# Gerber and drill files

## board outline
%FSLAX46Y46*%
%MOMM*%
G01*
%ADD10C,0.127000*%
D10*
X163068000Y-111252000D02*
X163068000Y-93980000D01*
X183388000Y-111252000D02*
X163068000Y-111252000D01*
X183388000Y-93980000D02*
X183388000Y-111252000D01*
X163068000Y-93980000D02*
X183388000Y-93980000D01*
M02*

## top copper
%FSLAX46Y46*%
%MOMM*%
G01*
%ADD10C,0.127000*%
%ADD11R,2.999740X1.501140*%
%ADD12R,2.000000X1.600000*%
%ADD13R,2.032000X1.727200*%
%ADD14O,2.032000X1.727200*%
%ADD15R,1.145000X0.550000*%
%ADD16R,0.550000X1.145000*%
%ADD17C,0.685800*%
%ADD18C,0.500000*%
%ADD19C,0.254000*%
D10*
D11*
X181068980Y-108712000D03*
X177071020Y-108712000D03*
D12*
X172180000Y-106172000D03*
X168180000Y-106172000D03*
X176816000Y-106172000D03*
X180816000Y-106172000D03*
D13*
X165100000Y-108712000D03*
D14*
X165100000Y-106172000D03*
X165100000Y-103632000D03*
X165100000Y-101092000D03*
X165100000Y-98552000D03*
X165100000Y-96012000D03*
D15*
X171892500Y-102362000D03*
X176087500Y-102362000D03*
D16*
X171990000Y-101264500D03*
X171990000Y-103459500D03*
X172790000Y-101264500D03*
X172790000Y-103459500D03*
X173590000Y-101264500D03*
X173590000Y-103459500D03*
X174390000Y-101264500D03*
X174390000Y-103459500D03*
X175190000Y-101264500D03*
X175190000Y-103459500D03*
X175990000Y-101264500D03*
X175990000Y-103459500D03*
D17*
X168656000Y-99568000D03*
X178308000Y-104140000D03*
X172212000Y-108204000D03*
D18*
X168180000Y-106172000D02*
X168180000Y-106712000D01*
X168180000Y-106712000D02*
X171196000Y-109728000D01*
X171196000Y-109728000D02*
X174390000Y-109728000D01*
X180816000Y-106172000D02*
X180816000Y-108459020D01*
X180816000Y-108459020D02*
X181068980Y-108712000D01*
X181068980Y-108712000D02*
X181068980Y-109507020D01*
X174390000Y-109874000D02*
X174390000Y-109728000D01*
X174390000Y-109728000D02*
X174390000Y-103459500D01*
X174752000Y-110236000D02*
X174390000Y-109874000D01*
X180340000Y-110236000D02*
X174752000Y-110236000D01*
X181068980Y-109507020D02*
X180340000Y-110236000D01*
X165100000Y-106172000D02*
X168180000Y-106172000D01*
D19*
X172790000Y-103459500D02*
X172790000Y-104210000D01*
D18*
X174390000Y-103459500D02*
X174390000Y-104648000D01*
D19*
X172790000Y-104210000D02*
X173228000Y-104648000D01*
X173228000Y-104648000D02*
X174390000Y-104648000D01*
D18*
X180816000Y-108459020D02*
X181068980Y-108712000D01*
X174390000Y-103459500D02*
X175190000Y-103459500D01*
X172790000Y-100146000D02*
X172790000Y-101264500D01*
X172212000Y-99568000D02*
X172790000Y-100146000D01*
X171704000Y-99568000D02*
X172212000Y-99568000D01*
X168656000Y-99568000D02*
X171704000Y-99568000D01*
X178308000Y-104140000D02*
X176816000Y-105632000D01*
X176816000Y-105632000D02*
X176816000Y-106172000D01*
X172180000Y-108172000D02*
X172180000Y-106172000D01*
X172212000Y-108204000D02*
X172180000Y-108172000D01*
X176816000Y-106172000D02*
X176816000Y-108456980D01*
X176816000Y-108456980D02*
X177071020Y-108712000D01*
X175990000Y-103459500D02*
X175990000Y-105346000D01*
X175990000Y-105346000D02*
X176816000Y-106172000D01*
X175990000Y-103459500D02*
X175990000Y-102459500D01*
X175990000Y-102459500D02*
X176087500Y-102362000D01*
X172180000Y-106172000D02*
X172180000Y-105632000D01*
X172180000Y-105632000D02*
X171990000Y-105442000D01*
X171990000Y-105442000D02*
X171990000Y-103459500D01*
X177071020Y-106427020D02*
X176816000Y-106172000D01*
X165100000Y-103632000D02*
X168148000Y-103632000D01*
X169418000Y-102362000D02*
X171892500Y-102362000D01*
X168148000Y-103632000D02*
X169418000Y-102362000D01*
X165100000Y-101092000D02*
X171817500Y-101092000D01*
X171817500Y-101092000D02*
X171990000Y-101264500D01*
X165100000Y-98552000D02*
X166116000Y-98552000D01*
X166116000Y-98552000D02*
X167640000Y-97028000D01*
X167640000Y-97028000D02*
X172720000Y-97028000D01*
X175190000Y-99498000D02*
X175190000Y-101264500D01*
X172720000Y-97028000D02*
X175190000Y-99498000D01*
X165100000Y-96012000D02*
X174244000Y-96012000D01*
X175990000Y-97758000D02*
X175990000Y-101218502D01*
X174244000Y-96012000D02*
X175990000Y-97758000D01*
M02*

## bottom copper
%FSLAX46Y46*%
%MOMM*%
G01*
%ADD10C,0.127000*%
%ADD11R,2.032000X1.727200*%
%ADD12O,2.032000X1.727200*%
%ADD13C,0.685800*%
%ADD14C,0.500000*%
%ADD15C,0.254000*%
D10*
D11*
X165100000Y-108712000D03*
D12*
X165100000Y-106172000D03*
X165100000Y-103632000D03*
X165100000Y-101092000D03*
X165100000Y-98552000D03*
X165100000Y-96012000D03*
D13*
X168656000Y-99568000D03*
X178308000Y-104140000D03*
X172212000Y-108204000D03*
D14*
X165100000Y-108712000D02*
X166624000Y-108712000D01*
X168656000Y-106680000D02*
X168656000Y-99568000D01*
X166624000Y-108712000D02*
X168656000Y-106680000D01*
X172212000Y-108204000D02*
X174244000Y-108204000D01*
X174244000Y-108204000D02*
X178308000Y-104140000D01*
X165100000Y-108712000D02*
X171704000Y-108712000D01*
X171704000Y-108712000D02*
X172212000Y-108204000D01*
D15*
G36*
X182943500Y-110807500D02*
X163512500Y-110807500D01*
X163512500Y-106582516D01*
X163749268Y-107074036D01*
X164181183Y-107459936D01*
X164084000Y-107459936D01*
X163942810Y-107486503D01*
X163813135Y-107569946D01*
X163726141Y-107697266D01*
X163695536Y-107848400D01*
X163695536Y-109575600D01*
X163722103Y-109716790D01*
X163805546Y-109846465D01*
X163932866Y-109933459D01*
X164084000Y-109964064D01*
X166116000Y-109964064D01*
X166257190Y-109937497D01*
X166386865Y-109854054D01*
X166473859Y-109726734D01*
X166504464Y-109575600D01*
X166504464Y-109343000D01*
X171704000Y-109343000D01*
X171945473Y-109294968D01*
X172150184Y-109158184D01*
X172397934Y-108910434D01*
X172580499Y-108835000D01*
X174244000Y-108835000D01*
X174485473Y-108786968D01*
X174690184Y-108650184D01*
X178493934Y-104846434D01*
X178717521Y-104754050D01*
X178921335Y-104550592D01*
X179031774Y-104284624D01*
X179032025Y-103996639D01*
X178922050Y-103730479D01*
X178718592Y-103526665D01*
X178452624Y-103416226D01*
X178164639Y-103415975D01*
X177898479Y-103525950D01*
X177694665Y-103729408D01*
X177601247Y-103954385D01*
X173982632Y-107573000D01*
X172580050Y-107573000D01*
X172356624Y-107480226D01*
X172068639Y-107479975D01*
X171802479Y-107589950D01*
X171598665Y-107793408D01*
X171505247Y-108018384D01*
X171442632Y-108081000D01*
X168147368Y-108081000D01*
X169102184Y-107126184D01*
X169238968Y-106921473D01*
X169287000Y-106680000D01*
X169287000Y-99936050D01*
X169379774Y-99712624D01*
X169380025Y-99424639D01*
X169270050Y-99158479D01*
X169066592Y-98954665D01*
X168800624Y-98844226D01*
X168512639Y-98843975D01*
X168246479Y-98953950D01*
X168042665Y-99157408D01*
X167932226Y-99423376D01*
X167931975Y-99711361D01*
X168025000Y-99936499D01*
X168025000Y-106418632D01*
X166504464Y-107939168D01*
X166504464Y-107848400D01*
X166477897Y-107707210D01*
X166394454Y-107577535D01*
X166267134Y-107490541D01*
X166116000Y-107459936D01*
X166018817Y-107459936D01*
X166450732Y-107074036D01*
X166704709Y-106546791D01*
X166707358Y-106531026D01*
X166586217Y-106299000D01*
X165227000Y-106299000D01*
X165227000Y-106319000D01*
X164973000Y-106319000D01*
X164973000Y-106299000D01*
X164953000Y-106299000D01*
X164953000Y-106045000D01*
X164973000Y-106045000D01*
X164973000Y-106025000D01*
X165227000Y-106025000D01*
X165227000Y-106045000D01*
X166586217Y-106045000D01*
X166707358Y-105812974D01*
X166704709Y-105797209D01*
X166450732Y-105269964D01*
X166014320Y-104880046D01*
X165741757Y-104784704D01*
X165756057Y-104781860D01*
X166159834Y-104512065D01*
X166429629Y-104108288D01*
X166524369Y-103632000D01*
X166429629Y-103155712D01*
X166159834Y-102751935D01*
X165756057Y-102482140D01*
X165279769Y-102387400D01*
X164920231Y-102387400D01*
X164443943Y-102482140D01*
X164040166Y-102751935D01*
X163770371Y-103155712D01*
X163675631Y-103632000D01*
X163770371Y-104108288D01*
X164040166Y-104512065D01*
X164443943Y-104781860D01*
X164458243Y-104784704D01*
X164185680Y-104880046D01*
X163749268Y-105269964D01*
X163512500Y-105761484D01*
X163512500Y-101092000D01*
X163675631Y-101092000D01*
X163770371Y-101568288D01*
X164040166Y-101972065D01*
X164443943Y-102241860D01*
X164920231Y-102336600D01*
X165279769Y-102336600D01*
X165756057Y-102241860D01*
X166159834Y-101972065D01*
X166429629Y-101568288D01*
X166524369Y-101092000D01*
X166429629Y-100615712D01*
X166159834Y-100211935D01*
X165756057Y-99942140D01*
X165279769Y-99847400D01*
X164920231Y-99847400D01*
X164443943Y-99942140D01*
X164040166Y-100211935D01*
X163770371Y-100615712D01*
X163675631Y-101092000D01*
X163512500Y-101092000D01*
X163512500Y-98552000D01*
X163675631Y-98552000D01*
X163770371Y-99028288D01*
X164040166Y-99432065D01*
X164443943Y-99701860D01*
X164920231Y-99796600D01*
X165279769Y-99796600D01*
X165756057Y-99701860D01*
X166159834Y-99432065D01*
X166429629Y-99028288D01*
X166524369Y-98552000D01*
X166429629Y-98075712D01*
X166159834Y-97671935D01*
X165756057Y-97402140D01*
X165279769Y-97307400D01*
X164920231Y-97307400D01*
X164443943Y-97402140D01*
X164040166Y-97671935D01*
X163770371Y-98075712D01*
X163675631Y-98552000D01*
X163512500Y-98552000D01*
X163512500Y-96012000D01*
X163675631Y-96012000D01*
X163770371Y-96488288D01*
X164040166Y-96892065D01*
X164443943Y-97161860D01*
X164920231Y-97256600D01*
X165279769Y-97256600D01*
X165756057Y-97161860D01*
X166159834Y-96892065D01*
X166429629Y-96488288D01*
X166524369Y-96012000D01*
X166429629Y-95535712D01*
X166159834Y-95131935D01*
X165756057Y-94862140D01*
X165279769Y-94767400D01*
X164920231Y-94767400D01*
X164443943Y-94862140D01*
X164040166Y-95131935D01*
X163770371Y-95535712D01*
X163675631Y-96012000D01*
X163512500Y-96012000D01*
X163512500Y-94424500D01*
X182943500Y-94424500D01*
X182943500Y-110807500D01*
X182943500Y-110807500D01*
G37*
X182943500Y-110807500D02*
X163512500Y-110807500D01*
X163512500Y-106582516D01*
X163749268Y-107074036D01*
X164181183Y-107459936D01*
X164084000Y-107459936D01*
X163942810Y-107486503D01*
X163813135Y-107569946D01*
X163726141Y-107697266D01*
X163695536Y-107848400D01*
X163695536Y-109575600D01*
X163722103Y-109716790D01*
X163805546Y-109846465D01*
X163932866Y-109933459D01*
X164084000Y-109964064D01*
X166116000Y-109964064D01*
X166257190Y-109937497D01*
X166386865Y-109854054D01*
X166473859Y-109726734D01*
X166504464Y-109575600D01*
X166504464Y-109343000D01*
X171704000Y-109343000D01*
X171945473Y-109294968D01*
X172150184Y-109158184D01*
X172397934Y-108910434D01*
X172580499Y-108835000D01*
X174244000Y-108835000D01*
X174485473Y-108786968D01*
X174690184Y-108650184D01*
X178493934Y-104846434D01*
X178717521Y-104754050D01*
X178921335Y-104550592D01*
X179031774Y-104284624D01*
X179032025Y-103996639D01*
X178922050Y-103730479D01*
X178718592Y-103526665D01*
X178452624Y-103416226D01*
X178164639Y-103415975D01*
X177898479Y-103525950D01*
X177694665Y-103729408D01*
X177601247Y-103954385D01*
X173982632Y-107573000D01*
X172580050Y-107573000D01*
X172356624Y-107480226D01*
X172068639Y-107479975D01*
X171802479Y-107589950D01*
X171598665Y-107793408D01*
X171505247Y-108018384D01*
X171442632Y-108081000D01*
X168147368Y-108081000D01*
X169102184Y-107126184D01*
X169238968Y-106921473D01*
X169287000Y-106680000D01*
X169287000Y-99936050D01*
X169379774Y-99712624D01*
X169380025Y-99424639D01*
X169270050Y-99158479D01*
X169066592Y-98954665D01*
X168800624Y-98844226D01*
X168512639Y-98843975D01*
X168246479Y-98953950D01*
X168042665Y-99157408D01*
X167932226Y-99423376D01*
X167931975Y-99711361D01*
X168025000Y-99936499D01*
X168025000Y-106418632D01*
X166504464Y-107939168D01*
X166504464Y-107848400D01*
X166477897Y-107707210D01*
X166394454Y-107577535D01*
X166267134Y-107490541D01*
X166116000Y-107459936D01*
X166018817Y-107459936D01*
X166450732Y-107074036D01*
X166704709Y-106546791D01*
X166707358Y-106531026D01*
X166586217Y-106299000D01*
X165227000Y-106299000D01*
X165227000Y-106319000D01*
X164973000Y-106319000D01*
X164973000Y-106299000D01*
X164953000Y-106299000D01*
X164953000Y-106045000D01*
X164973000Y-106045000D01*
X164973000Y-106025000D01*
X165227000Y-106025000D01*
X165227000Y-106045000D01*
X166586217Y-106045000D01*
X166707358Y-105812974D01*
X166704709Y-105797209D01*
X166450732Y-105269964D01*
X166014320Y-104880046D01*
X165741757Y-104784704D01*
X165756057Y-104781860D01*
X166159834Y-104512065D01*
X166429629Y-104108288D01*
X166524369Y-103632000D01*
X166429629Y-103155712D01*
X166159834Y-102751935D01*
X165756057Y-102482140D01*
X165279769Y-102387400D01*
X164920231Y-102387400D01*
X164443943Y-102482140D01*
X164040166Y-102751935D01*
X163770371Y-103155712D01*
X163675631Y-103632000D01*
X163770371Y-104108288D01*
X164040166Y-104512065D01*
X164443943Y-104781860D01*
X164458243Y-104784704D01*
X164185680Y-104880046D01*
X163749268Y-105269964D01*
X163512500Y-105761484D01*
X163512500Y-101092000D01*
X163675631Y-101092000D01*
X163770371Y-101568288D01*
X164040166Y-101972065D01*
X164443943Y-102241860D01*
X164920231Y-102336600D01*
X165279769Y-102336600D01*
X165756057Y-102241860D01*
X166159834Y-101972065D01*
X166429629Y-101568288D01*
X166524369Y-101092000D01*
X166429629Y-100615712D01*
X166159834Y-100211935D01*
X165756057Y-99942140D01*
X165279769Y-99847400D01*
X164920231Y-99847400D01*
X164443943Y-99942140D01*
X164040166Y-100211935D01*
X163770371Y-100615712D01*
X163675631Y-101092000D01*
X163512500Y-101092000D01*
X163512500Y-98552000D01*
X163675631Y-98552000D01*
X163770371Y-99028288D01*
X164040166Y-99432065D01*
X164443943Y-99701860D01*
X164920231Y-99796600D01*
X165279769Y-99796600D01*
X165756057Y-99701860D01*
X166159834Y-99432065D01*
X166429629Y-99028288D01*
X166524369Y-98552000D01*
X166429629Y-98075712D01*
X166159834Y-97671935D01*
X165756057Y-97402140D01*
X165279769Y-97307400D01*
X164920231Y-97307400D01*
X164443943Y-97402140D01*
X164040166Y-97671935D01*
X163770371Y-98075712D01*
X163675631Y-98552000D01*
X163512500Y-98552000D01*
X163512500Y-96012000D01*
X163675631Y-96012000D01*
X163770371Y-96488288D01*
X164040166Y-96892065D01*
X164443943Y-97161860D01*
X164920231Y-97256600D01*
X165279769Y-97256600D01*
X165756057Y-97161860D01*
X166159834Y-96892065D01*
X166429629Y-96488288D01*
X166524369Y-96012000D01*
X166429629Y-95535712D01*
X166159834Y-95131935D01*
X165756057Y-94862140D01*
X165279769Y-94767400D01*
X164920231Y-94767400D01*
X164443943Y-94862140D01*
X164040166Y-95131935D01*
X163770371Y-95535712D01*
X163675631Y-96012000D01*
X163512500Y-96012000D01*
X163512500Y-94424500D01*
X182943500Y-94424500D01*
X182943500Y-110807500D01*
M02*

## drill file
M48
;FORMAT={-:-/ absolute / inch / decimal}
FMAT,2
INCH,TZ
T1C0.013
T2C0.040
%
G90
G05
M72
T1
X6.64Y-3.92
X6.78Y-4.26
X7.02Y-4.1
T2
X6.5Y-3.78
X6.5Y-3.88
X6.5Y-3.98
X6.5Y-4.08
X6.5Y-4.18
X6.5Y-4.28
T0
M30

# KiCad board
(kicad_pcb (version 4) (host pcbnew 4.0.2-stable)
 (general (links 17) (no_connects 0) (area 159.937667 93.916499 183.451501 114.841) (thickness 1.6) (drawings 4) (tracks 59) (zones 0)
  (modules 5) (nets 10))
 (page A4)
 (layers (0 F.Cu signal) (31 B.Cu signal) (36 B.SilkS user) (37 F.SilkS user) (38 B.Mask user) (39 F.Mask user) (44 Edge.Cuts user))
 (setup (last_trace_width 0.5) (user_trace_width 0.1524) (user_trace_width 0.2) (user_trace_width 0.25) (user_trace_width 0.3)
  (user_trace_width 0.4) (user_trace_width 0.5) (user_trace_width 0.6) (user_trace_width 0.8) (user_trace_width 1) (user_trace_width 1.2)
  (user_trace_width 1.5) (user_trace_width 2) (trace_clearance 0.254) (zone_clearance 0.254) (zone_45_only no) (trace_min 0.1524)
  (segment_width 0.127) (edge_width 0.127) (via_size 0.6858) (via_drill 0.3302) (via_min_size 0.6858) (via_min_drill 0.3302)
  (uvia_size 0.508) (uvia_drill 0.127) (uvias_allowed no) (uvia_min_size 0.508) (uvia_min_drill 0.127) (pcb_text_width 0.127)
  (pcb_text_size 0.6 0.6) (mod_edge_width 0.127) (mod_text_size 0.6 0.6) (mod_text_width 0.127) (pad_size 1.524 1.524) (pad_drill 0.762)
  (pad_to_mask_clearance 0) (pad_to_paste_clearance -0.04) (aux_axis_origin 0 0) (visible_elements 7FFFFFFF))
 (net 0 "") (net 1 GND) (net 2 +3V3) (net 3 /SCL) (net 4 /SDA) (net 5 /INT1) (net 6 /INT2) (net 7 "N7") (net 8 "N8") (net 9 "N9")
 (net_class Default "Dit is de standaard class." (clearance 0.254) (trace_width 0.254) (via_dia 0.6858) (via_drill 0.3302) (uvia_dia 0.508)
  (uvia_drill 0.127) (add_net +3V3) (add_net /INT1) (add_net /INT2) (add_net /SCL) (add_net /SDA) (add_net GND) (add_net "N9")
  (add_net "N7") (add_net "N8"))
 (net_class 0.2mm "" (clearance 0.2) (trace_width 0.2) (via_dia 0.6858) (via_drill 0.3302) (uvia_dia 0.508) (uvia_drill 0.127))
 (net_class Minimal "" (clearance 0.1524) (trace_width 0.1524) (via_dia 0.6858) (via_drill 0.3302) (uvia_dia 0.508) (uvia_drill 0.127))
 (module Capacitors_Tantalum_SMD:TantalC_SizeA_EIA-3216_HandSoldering (layer F.Cu) (at 179.07 108.712)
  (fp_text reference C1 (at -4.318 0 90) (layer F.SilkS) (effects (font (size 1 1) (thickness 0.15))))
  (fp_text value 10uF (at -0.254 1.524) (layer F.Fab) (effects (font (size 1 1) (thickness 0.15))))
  (pad 2 smd rect (at 1.99898 0) (size 2.99974 1.50114) (layers F.Cu F.Mask) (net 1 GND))
  (pad 1 smd rect (at -1.99898 0) (size 2.99974 1.50114) (layers F.Cu F.Mask) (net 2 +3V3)))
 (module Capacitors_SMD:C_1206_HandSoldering (layer F.Cu) (at 170.18 106.172 180)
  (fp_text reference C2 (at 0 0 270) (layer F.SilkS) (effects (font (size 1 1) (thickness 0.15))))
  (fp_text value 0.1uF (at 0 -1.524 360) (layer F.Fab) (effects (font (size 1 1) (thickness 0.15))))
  (pad 1 smd rect (at -2 0 180) (size 2 1.6) (layers F.Cu F.Mask) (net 2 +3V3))
  (pad 2 smd rect (at 2 0 180) (size 2 1.6) (layers F.Cu F.Mask) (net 1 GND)))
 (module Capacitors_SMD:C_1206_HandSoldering (layer F.Cu) (at 178.816 106.172)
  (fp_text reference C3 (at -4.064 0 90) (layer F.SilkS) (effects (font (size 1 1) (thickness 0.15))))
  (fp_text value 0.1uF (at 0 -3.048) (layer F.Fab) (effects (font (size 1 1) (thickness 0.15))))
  (pad 1 smd rect (at -2 0) (size 2 1.6) (layers F.Cu F.Mask) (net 2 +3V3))
  (pad 2 smd rect (at 2 0) (size 2 1.6) (layers F.Cu F.Mask) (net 1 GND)))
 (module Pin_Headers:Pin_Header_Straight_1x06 (layer F.Cu) (at 165.1 108.712 180)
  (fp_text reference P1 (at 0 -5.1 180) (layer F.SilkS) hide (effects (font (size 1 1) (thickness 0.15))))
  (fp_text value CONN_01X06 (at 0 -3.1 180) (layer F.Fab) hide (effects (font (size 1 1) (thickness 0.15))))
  (pad 1 thru_hole rect (at 0 0 180) (size 2.032 1.7272) (drill 1.016) (layers *.Cu *.Mask F.SilkS) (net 2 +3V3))
  (pad 2 thru_hole oval (at 0 2.54 180) (size 2.032 1.7272) (drill 1.016) (layers *.Cu *.Mask F.SilkS) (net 1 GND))
  (pad 3 thru_hole oval (at 0 5.08 180) (size 2.032 1.7272) (drill 1.016) (layers *.Cu *.Mask F.SilkS) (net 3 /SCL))
  (pad 4 thru_hole oval (at 0 7.62 180) (size 2.032 1.7272) (drill 1.016) (layers *.Cu *.Mask F.SilkS) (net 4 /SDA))
  (pad 5 thru_hole oval (at 0 10.16 180) (size 2.032 1.7272) (drill 1.016) (layers *.Cu *.Mask F.SilkS) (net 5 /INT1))
  (pad 6 thru_hole oval (at 0 12.7 180) (size 2.032 1.7272) (drill 1.016) (layers *.Cu *.Mask F.SilkS) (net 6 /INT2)))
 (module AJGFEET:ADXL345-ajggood (layer F.Cu) (at 173.99 102.362)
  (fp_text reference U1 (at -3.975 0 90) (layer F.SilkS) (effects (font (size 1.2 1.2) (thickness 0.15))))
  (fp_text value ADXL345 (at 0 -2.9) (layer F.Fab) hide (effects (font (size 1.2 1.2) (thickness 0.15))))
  (pad 14 smd rect (at -2.0975 0) (size 1.145 0.55) (layers F.Cu F.Mask) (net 3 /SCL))
  (pad 7 smd rect (at 2.0975 0) (size 1.145 0.55) (layers F.Cu F.Mask) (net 2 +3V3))
  (pad 13 smd rect (at -2 -1.0975) (size 0.55 1.145) (layers F.Cu F.Mask) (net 4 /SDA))
  (pad 1 smd rect (at -2 1.0975) (size 0.55 1.145) (layers F.Cu F.Mask) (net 2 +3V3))
  (pad 12 smd rect (at -1.2 -1.0975) (size 0.55 1.145) (layers F.Cu F.Mask) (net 2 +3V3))
  (pad 2 smd rect (at -1.2 1.0975) (size 0.55 1.145) (layers F.Cu F.Mask) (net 1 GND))
  (pad 11 smd rect (at -0.4 -1.0975) (size 0.55 1.145) (layers F.Cu F.Mask) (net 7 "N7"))
  (pad 3 smd rect (at -0.4 1.0975) (size 0.55 1.145) (layers F.Cu F.Mask) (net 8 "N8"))
  (pad 10 smd rect (at 0.4 -1.0975) (size 0.55 1.145) (layers F.Cu F.Mask) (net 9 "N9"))
  (pad 4 smd rect (at 0.4 1.0975) (size 0.55 1.145) (layers F.Cu F.Mask) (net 1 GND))
  (pad 9 smd rect (at 1.2 -1.0975) (size 0.55 1.145) (layers F.Cu F.Mask) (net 5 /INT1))
  (pad 5 smd rect (at 1.2 1.0975) (size 0.55 1.145) (layers F.Cu F.Mask) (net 1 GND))
  (pad 8 smd rect (at 2 -1.0975) (size 0.55 1.145) (layers F.Cu F.Mask) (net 6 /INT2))
  (pad 6 smd rect (at 2 1.0975) (size 0.55 1.145) (layers F.Cu F.Mask) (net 2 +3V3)))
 (gr_line (start 163.068 111.252) (end 163.068 93.98) (angle 90) (layer Edge.Cuts) (width 0.127))
 (gr_line (start 183.388 111.252) (end 163.068 111.252) (angle 90) (layer Edge.Cuts) (width 0.127))
 (gr_line (start 183.388 93.98) (end 183.388 111.252) (angle 90) (layer Edge.Cuts) (width 0.127))
 (gr_line (start 163.068 93.98) (end 183.388 93.98) (angle 90) (layer Edge.Cuts) (width 0.127))
 (segment (start 168.18 106.172) (end 168.18 106.712) (width 0.5) (layer F.Cu) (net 1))
 (segment (start 168.18 106.712) (end 171.196 109.728) (width 0.5) (layer F.Cu) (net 1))
 (segment (start 171.196 109.728) (end 174.39 109.728) (width 0.5) (layer F.Cu) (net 1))
 (segment (start 180.816 106.172) (end 180.816 108.45902) (width 0.5) (layer F.Cu) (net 1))
 (segment (start 180.816 108.45902) (end 181.06898 108.712) (width 0.5) (layer F.Cu) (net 1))
 (segment (start 181.06898 108.712) (end 181.06898 109.50702) (width 0.5) (layer F.Cu) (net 1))
 (segment (start 174.39 109.874) (end 174.39 109.728) (width 0.5) (layer F.Cu) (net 1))
 (segment (start 174.39 109.728) (end 174.39 103.4595) (width 0.5) (layer F.Cu) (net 1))
 (segment (start 174.752 110.236) (end 174.39 109.874) (width 0.5) (layer F.Cu) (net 1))
 (segment (start 180.34 110.236) (end 174.752 110.236) (width 0.5) (layer F.Cu) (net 1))
 (segment (start 181.06898 109.50702) (end 180.34 110.236) (width 0.5) (layer F.Cu) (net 1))
 (segment (start 165.1 106.172) (end 168.18 106.172) (width 0.5) (layer F.Cu) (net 1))
 (segment (start 172.79 103.4595) (end 172.79 104.21) (width 0.254) (layer F.Cu) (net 1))
 (segment (start 174.39 103.4595) (end 174.39 104.648) (width 0.5) (layer F.Cu) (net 1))
 (segment (start 172.79 104.21) (end 173.228 104.648) (width 0.254) (layer F.Cu) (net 1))
 (segment (start 173.228 104.648) (end 174.39 104.648) (width 0.254) (layer F.Cu) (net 1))
 (segment (start 180.816 108.45902) (end 181.06898 108.712) (width 0.5) (layer F.Cu) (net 1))
 (segment (start 174.39 103.4595) (end 175.19 103.4595) (width 0.5) (layer F.Cu) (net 1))
 (segment (start 165.1 108.712) (end 166.624 108.712) (width 0.5) (layer B.Cu) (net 2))
 (segment (start 172.79 100.146) (end 172.79 101.2645) (width 0.5) (layer F.Cu) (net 2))
 (segment (start 172.212 99.568) (end 172.79 100.146) (width 0.5) (layer F.Cu) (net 2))
 (segment (start 171.704 99.568) (end 172.212 99.568) (width 0.5) (layer F.Cu) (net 2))
 (segment (start 168.656 99.568) (end 171.704 99.568) (width 0.5) (layer F.Cu) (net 2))
 (via (at 168.656 99.568) (size 0.6858) (drill 0.3302) (layers F.Cu B.Cu) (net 2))
 (segment (start 168.656 106.68) (end 168.656 99.568) (width 0.5) (layer B.Cu) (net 2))
 (segment (start 166.624 108.712) (end 168.656 106.68) (width 0.5) (layer B.Cu) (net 2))
 (segment (start 172.212 108.204) (end 174.244 108.204) (width 0.5) (layer B.Cu) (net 2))
 (segment (start 178.308 104.14) (end 176.816 105.632) (width 0.5) (layer F.Cu) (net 2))
 (via (at 178.308 104.14) (size 0.6858) (drill 0.3302) (layers F.Cu B.Cu) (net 2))
 (segment (start 174.244 108.204) (end 178.308 104.14) (width 0.5) (layer B.Cu) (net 2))
 (segment (start 176.816 105.632) (end 176.816 106.172) (width 0.5) (layer F.Cu) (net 2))
 (segment (start 165.1 108.712) (end 171.704 108.712) (width 0.5) (layer B.Cu) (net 2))
 (segment (start 172.18 108.172) (end 172.18 106.172) (width 0.5) (layer F.Cu) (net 2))
 (segment (start 172.212 108.204) (end 172.18 108.172) (width 0.5) (layer F.Cu) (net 2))
 (via (at 172.212 108.204) (size 0.6858) (drill 0.3302) (layers F.Cu B.Cu) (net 2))
 (segment (start 171.704 108.712) (end 172.212 108.204) (width 0.5) (layer B.Cu) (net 2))
 (segment (start 176.816 106.172) (end 176.816 108.45698) (width 0.5) (layer F.Cu) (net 2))
 (segment (start 176.816 108.45698) (end 177.07102 108.712) (width 0.5) (layer F.Cu) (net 2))
 (segment (start 175.99 103.4595) (end 175.99 105.346) (width 0.5) (layer F.Cu) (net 2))
 (segment (start 175.99 105.346) (end 176.816 106.172) (width 0.5) (layer F.Cu) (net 2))
 (segment (start 175.99 103.4595) (end 175.99 102.4595) (width 0.5) (layer F.Cu) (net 2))
 (segment (start 175.99 102.4595) (end 176.0875 102.362) (width 0.5) (layer F.Cu) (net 2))
 (segment (start 172.18 106.172) (end 172.18 105.632) (width 0.5) (layer F.Cu) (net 2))
 (segment (start 172.18 105.632) (end 171.99 105.442) (width 0.5) (layer F.Cu) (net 2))
 (segment (start 171.99 105.442) (end 171.99 103.4595) (width 0.5) (layer F.Cu) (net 2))
 (segment (start 177.07102 106.42702) (end 176.816 106.172) (width 0.5) (layer F.Cu) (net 2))
 (segment (start 165.1 103.632) (end 168.148 103.632) (width 0.5) (layer F.Cu) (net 3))
 (segment (start 169.418 102.362) (end 171.8925 102.362) (width 0.5) (layer F.Cu) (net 3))
 (segment (start 168.148 103.632) (end 169.418 102.362) (width 0.5) (layer F.Cu) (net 3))
 (segment (start 165.1 101.092) (end 171.8175 101.092) (width 0.5) (layer F.Cu) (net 4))
 (segment (start 171.8175 101.092) (end 171.99 101.2645) (width 0.5) (layer F.Cu) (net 4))
 (segment (start 165.1 98.552) (end 166.116 98.552) (width 0.5) (layer F.Cu) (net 5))
 (segment (start 166.116 98.552) (end 167.64 97.028) (width 0.5) (layer F.Cu) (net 5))
 (segment (start 167.64 97.028) (end 172.72 97.028) (width 0.5) (layer F.Cu) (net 5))
 (segment (start 175.19 99.498) (end 175.19 101.2645) (width 0.5) (layer F.Cu) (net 5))
 (segment (start 172.72 97.028) (end 175.19 99.498) (width 0.5) (layer F.Cu) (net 5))
 (segment (start 165.1 96.012) (end 174.244 96.012) (width 0.5) (layer F.Cu) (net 6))
 (segment (start 175.99 97.758) (end 175.99 101.218502) (width 0.5) (layer F.Cu) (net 6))
 (segment (start 174.244 96.012) (end 175.99 97.758) (width 0.5) (layer F.Cu) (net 6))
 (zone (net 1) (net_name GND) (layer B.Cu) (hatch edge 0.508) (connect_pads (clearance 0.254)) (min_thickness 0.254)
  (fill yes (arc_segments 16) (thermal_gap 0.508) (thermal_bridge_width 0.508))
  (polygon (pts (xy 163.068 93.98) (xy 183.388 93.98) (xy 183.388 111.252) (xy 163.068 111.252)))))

